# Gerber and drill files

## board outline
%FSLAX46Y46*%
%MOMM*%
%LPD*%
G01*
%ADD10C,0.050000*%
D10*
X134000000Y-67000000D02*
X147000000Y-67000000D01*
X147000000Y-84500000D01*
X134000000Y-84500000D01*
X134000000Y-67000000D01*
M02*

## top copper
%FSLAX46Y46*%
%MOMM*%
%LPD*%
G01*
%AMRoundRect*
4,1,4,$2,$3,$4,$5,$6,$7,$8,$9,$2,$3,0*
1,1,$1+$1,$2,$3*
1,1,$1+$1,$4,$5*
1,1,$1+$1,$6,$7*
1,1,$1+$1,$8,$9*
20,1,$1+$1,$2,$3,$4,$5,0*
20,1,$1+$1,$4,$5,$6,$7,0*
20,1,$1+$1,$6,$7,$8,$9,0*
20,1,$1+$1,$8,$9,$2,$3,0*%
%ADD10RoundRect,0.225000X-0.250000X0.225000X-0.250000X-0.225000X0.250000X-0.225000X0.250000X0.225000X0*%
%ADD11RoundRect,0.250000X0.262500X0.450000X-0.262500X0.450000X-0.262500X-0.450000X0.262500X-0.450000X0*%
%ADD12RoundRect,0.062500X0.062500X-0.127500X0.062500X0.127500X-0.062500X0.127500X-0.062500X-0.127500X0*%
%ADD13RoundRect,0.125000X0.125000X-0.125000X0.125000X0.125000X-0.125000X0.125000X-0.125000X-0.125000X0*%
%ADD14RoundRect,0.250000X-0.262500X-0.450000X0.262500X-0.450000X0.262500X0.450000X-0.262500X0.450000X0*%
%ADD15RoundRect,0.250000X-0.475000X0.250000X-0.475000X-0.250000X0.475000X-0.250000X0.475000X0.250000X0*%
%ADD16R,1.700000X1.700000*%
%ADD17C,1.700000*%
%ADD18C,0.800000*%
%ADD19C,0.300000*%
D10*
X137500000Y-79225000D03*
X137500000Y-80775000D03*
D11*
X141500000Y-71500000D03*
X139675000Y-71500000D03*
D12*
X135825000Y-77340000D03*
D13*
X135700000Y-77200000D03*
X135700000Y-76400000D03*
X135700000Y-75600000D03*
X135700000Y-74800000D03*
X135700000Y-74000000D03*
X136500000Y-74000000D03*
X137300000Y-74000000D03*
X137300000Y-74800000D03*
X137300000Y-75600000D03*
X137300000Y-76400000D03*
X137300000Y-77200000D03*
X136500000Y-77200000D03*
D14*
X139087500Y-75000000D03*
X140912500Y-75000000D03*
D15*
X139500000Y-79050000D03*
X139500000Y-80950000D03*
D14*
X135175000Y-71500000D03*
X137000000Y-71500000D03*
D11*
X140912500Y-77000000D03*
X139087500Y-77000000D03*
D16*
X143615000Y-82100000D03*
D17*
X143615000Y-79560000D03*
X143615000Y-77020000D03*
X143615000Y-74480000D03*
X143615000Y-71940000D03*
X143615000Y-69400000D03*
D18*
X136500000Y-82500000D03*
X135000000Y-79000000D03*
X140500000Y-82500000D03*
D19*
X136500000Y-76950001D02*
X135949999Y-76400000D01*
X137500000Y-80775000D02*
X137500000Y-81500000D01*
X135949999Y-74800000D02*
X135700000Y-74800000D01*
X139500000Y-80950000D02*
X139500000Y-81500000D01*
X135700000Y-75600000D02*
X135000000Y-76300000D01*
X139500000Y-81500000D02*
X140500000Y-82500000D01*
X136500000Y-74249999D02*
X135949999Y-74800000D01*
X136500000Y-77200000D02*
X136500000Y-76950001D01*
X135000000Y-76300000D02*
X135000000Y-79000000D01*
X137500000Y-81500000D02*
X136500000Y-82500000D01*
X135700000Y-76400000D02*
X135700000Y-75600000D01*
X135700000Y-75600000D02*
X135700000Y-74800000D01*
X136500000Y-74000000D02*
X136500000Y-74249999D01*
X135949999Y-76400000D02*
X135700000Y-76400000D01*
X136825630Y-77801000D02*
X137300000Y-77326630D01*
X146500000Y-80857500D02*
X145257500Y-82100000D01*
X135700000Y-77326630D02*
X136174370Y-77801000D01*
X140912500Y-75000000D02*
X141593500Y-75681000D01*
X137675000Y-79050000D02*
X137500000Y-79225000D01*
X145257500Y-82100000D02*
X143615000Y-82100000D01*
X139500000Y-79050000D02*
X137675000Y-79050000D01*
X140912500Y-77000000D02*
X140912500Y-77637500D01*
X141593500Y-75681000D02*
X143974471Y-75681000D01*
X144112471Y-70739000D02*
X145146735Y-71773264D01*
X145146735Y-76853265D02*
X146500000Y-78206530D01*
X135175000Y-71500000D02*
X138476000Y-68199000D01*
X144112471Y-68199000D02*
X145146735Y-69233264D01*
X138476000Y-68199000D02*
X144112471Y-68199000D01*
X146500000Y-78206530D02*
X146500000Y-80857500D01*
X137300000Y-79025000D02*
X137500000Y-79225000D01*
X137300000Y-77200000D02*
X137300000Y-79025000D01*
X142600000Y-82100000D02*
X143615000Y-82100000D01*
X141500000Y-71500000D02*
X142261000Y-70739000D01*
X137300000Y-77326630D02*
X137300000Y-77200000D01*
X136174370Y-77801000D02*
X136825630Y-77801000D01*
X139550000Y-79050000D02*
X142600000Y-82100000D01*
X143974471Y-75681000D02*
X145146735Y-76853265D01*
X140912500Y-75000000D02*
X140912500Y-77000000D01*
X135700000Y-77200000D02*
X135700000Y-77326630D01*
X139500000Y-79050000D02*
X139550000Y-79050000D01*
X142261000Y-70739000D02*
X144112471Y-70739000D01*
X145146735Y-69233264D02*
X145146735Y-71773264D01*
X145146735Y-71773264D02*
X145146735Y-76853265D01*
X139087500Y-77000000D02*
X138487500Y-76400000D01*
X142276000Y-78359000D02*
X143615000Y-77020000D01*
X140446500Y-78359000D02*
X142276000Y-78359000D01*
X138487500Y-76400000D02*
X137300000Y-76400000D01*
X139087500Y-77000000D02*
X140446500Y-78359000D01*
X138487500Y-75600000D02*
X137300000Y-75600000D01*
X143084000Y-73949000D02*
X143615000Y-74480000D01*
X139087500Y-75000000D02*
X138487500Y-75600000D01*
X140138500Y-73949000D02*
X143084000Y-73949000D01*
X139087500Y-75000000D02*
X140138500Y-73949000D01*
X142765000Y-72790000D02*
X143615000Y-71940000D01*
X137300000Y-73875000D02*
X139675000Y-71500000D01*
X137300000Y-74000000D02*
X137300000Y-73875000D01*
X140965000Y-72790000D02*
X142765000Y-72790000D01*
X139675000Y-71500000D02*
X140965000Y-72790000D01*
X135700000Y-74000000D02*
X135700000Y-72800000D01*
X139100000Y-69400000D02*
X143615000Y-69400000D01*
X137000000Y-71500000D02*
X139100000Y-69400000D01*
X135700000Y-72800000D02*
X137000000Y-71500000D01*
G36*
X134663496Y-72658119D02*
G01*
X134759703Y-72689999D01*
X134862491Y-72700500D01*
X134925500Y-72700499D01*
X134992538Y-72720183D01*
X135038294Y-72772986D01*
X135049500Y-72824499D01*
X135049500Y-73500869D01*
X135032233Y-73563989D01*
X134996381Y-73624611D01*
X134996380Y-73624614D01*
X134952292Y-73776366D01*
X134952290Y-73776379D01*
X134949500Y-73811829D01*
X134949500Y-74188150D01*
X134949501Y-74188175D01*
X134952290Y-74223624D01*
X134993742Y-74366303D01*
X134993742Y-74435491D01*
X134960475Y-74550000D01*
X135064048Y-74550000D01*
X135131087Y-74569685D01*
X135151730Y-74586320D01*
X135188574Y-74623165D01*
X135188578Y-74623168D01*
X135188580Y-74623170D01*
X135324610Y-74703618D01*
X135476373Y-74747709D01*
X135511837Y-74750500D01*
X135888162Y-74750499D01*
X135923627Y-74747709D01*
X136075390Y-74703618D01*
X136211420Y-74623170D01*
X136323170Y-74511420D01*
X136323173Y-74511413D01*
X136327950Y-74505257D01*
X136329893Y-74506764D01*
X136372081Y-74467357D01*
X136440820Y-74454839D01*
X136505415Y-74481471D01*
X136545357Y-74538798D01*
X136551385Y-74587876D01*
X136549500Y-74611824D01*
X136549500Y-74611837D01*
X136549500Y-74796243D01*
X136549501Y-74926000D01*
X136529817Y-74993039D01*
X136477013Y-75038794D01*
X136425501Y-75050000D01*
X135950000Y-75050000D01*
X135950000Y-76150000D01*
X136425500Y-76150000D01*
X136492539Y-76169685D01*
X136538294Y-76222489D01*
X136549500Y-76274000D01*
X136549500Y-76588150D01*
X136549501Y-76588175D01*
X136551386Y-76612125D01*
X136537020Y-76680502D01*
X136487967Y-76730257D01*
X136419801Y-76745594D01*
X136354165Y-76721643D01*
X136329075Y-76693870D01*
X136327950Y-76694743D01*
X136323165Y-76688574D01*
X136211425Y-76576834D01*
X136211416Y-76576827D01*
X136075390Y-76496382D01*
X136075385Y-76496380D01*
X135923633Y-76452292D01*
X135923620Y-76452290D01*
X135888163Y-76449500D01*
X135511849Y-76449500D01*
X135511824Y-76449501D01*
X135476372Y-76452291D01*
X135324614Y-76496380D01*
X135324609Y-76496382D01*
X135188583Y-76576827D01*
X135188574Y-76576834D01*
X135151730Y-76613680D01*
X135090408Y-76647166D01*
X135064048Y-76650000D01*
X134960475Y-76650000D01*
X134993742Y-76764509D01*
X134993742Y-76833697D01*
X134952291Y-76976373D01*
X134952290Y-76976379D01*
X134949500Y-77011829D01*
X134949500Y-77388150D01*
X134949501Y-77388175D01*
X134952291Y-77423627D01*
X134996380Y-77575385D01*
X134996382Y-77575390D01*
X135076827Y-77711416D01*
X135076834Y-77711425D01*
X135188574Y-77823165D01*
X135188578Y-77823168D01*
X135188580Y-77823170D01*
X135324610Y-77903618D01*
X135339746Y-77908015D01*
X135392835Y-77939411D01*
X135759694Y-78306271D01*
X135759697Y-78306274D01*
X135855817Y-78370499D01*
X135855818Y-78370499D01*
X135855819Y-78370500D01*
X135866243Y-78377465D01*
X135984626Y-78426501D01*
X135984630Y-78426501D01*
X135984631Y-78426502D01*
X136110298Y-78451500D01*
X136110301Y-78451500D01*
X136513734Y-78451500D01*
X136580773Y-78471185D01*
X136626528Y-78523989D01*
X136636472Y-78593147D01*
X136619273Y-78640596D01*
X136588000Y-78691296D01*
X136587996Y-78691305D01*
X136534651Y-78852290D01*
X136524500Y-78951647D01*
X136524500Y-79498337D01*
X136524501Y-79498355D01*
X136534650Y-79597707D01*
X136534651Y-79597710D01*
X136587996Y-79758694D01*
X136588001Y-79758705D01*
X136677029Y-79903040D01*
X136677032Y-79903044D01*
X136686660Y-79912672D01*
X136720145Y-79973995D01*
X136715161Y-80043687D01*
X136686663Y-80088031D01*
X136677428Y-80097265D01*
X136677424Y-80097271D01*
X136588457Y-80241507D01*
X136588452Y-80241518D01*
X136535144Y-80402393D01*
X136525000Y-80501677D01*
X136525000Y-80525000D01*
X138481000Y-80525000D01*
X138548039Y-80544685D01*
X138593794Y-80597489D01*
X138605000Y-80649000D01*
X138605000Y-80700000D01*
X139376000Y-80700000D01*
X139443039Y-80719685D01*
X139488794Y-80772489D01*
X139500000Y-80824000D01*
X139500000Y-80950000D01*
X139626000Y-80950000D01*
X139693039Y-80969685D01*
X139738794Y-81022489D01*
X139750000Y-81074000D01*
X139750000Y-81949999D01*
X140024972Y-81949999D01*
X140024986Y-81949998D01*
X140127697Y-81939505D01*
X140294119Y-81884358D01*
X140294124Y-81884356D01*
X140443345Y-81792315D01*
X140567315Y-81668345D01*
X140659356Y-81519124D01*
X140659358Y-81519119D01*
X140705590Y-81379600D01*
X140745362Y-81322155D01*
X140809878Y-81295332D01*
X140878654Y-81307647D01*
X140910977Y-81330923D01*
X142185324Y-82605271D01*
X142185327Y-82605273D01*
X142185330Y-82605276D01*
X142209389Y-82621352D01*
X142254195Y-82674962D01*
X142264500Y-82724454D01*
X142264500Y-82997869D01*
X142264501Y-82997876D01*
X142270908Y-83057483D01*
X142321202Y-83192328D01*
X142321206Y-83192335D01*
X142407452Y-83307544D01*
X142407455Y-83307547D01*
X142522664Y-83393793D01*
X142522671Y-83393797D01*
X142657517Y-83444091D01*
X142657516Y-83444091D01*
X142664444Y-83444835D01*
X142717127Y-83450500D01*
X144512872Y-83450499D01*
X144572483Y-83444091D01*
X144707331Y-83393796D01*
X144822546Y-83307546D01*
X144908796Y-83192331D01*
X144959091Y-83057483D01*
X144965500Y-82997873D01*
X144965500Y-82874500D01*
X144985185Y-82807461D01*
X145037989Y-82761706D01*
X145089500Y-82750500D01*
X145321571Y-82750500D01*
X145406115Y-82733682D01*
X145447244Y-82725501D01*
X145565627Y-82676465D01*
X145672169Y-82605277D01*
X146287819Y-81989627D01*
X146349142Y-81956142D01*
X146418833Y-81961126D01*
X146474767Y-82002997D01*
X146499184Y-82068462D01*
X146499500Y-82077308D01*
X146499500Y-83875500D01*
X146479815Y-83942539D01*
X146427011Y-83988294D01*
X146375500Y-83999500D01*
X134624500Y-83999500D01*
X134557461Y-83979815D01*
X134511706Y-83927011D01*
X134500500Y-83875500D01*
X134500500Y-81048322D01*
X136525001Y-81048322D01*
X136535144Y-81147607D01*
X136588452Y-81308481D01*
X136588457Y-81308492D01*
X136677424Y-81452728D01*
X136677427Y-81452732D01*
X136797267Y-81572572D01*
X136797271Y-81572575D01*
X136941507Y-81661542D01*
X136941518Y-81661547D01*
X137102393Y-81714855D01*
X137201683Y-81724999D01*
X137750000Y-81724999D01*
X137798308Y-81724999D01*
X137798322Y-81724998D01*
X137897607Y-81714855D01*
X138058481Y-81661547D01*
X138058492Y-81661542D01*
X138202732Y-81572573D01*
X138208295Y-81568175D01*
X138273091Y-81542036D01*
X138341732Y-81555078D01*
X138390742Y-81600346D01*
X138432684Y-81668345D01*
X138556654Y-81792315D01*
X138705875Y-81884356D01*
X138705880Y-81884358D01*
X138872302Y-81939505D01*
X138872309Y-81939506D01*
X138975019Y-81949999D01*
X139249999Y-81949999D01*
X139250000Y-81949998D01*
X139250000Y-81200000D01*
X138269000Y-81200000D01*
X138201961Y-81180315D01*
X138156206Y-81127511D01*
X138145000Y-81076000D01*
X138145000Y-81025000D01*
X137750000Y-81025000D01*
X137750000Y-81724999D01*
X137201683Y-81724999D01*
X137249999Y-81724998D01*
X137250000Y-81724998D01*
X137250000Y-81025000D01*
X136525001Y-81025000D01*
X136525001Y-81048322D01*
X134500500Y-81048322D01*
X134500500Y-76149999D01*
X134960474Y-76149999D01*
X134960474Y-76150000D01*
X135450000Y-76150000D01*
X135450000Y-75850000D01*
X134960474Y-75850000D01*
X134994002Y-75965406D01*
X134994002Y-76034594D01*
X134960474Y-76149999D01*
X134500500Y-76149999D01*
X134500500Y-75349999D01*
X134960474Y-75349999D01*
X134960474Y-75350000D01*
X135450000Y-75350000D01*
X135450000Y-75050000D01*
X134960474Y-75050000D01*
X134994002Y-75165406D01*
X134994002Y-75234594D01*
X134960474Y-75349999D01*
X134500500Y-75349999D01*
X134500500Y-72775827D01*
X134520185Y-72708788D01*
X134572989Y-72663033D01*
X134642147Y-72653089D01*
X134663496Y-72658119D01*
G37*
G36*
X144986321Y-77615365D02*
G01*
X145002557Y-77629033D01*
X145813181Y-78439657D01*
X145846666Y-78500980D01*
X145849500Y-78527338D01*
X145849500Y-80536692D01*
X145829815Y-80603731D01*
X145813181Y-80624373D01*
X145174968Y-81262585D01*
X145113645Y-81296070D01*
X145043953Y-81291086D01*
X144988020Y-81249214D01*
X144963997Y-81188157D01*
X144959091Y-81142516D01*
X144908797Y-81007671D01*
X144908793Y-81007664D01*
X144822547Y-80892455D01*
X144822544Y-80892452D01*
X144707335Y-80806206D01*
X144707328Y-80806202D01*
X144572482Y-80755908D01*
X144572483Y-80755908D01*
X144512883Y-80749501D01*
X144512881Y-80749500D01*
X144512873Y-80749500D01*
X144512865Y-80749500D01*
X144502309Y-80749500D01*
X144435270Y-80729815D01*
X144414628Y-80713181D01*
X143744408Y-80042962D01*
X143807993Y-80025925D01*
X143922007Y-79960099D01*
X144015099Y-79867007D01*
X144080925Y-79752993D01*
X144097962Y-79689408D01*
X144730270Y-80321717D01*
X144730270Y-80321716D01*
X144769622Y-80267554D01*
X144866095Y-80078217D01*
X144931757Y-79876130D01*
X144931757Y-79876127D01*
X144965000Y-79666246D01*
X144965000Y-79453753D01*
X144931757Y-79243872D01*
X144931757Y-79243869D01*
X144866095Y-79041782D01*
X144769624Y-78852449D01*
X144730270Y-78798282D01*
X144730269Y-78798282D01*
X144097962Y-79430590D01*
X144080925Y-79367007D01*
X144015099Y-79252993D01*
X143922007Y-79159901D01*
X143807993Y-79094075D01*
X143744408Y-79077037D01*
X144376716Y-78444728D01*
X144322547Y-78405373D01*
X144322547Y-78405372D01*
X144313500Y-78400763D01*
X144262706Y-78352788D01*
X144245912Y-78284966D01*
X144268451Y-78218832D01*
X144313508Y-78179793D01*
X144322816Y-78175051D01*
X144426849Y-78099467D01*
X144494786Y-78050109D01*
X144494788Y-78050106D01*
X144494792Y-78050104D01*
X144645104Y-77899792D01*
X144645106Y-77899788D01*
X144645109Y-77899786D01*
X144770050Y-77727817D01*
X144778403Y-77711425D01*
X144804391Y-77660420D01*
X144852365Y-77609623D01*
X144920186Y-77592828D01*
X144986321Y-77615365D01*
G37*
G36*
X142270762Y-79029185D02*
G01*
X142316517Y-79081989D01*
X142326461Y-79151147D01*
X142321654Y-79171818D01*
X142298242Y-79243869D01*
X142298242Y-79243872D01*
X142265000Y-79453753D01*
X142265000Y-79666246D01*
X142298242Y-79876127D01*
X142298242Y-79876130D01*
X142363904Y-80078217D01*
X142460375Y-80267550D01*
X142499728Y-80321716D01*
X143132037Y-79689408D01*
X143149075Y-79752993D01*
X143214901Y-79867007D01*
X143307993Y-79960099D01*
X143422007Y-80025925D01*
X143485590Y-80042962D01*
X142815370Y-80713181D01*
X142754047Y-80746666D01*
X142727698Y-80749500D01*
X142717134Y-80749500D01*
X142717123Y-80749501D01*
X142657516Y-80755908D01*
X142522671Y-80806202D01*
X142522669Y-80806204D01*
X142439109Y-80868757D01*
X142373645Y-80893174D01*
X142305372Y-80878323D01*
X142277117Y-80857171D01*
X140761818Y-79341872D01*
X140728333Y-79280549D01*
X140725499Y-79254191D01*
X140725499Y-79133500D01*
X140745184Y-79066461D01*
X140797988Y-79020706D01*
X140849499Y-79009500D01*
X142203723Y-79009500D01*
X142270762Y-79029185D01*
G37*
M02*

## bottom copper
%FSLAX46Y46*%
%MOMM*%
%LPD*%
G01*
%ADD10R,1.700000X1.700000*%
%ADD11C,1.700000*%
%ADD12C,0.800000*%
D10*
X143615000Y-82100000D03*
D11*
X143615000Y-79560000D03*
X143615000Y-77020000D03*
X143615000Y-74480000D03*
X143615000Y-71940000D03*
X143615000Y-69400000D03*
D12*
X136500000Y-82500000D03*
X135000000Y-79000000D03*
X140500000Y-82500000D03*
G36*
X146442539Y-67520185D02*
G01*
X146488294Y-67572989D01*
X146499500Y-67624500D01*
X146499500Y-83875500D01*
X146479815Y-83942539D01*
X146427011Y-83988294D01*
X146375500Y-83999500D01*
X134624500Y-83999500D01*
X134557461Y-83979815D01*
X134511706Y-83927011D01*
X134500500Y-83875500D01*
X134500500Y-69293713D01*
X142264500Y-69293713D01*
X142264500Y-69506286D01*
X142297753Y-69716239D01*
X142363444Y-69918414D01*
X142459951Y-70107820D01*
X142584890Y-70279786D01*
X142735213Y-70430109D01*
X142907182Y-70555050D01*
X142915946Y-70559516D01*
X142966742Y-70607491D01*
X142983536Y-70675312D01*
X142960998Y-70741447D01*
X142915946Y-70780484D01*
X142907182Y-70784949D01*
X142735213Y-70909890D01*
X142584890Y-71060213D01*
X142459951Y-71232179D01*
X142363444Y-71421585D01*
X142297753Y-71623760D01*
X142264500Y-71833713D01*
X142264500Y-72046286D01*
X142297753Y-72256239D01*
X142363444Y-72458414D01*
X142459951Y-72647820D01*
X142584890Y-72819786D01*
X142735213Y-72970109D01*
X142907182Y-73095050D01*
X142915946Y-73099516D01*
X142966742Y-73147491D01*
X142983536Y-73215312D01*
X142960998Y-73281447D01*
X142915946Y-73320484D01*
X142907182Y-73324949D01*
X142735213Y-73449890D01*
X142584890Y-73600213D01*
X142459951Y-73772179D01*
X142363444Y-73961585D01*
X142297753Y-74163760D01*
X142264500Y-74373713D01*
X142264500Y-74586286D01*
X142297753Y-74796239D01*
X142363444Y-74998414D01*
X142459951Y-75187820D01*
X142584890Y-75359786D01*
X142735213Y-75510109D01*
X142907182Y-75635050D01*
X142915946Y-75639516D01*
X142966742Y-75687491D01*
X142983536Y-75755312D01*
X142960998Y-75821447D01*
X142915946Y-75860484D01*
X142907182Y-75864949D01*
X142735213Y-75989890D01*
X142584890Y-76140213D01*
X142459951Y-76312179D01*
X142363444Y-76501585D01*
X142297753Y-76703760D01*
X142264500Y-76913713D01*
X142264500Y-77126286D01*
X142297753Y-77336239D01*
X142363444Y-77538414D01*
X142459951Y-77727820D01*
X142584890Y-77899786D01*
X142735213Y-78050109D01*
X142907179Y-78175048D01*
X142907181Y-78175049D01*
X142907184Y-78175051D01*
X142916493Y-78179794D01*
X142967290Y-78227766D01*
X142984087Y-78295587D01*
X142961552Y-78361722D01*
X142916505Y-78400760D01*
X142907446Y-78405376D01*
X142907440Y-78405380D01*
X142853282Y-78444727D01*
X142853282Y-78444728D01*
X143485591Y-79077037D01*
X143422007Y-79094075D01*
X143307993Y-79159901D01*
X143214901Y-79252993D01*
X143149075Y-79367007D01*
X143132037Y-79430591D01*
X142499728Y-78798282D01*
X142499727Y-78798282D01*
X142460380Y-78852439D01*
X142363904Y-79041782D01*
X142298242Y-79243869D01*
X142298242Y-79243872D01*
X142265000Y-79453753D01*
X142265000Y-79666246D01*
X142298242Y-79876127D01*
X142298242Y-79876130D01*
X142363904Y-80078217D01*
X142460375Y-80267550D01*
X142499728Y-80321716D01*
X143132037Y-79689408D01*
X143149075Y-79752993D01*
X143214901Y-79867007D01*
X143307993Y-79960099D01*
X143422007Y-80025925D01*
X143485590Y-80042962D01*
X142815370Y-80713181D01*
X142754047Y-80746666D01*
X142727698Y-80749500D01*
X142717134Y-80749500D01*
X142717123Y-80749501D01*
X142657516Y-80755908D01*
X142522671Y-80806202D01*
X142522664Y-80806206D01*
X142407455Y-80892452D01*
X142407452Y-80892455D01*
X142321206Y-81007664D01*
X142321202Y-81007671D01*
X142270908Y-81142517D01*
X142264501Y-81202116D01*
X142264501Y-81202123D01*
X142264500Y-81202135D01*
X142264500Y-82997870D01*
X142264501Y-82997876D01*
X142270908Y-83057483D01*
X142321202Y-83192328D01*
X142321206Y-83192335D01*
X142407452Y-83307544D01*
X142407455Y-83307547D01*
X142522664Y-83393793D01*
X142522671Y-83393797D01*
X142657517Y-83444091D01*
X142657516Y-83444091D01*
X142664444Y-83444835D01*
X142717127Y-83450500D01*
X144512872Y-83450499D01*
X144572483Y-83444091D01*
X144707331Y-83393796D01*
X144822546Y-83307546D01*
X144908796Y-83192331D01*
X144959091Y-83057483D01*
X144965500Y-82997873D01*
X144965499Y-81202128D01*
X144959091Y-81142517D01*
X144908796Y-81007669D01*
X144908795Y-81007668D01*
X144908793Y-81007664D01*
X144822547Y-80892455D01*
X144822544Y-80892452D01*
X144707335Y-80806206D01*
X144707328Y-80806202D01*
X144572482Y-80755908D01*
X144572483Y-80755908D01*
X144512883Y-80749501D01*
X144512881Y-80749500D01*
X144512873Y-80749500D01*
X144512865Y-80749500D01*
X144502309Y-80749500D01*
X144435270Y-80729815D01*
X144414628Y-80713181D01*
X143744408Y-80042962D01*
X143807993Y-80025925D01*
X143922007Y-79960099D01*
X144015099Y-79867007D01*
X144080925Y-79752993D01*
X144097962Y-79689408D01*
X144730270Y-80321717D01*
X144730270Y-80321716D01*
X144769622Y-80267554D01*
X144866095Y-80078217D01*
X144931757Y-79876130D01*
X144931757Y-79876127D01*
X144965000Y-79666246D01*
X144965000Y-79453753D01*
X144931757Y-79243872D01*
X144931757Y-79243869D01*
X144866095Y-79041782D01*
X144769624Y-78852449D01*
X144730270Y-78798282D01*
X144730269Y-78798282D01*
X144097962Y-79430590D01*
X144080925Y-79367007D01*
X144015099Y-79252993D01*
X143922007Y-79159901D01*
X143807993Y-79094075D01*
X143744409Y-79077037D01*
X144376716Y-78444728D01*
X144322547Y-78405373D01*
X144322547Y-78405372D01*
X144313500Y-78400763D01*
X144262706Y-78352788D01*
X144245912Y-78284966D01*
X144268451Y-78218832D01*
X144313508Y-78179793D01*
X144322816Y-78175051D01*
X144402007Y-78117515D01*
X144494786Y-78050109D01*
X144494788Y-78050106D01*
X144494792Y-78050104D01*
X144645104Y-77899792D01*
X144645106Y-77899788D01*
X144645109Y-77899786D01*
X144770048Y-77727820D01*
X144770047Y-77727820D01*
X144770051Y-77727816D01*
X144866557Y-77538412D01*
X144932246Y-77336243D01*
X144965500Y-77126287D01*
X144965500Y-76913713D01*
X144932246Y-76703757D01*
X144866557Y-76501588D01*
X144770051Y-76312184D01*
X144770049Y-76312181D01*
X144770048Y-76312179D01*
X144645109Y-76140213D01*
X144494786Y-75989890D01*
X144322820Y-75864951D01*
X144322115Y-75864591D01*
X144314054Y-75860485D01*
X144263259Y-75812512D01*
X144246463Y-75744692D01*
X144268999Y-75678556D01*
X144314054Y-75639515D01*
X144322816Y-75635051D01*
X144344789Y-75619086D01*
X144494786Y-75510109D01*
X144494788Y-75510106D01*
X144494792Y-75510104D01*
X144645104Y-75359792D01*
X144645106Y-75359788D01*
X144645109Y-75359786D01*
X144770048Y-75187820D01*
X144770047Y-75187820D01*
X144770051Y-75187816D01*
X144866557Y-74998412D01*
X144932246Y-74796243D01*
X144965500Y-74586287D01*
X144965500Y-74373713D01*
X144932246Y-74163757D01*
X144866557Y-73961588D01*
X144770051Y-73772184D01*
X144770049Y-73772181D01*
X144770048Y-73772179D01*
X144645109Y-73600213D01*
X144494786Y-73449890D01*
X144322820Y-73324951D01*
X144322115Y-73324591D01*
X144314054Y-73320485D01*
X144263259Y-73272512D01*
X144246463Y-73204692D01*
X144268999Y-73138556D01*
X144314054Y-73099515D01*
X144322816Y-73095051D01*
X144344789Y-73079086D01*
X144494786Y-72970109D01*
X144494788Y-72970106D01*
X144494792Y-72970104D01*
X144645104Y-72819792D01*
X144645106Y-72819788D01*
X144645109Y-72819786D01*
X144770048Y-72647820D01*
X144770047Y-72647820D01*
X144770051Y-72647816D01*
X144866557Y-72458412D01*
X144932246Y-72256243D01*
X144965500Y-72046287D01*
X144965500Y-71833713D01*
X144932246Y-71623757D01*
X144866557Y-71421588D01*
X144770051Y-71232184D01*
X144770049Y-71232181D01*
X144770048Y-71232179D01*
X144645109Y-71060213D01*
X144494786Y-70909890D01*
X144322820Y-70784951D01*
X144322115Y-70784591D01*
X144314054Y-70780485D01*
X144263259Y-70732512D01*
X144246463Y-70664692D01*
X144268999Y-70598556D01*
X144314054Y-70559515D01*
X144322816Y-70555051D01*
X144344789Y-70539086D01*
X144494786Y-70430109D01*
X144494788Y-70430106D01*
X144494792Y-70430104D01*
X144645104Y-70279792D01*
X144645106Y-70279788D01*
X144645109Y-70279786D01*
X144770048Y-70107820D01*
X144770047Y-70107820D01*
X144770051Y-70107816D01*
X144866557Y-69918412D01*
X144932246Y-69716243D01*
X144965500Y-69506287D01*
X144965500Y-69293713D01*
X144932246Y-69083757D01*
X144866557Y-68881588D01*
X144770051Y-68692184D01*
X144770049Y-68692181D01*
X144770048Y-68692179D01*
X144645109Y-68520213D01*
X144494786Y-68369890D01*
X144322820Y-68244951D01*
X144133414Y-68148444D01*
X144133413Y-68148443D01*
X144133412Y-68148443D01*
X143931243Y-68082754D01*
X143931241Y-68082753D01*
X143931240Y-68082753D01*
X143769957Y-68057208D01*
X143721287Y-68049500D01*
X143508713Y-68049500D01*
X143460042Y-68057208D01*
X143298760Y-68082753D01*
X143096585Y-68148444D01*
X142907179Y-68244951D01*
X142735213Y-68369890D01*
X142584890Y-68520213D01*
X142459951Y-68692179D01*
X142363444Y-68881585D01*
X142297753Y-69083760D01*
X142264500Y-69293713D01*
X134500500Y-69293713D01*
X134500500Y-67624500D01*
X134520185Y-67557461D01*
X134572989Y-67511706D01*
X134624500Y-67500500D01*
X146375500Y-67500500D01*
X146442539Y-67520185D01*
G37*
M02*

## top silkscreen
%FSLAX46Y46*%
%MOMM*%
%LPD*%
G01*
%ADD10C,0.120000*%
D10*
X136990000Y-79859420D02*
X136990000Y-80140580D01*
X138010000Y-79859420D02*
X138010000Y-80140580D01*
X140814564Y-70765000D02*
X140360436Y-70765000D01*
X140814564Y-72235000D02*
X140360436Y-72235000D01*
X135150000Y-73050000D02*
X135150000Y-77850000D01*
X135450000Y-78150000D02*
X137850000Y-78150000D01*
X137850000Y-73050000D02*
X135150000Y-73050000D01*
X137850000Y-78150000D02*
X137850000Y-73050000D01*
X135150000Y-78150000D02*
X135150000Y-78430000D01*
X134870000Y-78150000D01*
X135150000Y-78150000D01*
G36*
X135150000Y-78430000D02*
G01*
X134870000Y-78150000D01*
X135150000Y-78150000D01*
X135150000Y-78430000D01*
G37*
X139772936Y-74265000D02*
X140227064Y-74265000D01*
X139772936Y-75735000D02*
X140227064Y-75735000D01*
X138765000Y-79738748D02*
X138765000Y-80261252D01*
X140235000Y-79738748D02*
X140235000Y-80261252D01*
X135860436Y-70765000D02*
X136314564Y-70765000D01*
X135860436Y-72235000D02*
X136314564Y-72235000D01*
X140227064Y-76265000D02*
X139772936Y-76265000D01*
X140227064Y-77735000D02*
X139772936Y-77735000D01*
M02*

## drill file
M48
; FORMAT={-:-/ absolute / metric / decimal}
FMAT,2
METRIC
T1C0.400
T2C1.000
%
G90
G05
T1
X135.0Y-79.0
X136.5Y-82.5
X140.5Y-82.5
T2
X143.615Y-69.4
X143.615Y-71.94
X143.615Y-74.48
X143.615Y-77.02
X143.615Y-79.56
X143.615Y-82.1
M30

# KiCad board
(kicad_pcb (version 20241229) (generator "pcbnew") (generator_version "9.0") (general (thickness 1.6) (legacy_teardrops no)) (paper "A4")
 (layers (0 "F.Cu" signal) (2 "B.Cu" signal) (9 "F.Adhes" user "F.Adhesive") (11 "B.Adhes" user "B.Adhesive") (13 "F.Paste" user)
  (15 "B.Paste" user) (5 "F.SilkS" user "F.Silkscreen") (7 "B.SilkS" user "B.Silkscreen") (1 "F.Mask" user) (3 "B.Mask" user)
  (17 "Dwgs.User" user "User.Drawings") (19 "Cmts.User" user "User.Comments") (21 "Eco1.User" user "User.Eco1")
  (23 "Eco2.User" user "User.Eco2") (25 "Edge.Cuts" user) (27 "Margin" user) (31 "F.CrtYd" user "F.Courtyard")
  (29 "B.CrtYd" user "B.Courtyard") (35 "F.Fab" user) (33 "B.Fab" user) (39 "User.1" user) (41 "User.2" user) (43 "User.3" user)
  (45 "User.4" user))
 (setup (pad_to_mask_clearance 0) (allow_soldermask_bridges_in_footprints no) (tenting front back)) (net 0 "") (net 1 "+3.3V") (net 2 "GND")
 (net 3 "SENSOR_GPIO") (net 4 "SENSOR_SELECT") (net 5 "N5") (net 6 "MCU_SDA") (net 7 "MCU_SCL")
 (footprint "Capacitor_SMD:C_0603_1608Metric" (layer "F.Cu") (at 137.5 80 -90)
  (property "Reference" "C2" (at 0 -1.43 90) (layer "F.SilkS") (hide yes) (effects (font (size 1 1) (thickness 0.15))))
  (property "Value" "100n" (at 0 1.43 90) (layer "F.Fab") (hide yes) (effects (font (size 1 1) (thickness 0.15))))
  (fp_line (start -0.14058 0.51) (end 0.14058 0.51) (stroke (width 0.12) (type solid)) (layer "F.SilkS"))
  (fp_line (start -0.14058 -0.51) (end 0.14058 -0.51) (stroke (width 0.12) (type solid)) (layer "F.SilkS"))
  (pad "1" smd roundrect (at -0.775 0 270) (size 0.9 0.95) (layers "F.Cu" "F.Mask" "F.Paste") (roundrect_rratio 0.25) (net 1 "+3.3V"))
  (pad "2" smd roundrect (at 0.775 0 270) (size 0.9 0.95) (layers "F.Cu" "F.Mask" "F.Paste") (roundrect_rratio 0.25) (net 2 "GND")))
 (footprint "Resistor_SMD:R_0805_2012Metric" (layer "F.Cu") (at 140.5875 71.5 180)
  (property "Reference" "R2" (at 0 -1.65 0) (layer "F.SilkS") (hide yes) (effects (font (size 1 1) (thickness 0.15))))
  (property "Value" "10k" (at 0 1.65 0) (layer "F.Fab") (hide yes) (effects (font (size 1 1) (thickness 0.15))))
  (fp_line (start -0.227064 0.735) (end 0.227064 0.735) (stroke (width 0.12) (type solid)) (layer "F.SilkS"))
  (fp_line (start -0.227064 -0.735) (end 0.227064 -0.735) (stroke (width 0.12) (type solid)) (layer "F.SilkS"))
  (pad "1" smd roundrect (at -0.9125 0 180) (size 1.025 1.4) (layers "F.Cu" "F.Mask" "F.Paste") (roundrect_rratio 0.243902) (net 1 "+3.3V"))
  (pad "2" smd roundrect (at 0.9125 0 180) (size 1.025 1.4) (layers "F.Cu" "F.Mask" "F.Paste") (roundrect_rratio 0.243902)
   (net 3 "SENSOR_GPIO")))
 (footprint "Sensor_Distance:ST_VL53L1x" (layer "F.Cu") (at 136.5 75.6 90)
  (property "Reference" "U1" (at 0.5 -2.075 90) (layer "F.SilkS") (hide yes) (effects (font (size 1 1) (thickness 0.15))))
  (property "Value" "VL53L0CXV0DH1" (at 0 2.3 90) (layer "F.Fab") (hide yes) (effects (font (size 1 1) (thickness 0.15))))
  (fp_line (start 2.55 -1.35) (end -2.25 -1.35) (stroke (width 0.12) (type solid)) (layer "F.SilkS"))
  (fp_line (start -2.55 -1.05) (end -2.55 1.35) (stroke (width 0.12) (type solid)) (layer "F.SilkS"))
  (fp_line (start 2.55 1.35) (end 2.55 -1.35) (stroke (width 0.12) (type solid)) (layer "F.SilkS"))
  (fp_line (start -2.55 1.35) (end 2.55 1.35) (stroke (width 0.12) (type solid)) (layer "F.SilkS"))
  (fp_poly
   (pts (xy -2.55 -1.35) (xy -2.83 -1.35) (xy -2.55 -1.63) (xy -2.55 -1.35)) (stroke (width 0.12) (type solid)) (fill yes) (layer "F.SilkS"))
  (pad "1" smd roundrect (at -1.74 -0.675 90) (size 0.38 0.25) (layers "F.Cu" "F.Mask" "F.Paste") (roundrect_rratio 0.25) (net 1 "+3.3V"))
  (pad "1" smd roundrect (at -1.6 -0.8 90) (size 0.5 0.5) (layers "F.Cu" "F.Mask" "F.Paste") (roundrect_rratio 0.25) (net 1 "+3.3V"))
  (pad "2" smd roundrect (at -0.8 -0.8 90) (size 0.5 0.5) (layers "F.Cu" "F.Mask" "F.Paste") (roundrect_rratio 0.25) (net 2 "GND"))
  (pad "3" smd roundrect (at 0 -0.8 90) (size 0.5 0.5) (layers "F.Cu" "F.Mask" "F.Paste") (roundrect_rratio 0.25) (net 2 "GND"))
  (pad "4" smd roundrect (at 0.8 -0.8 90) (size 0.5 0.5) (layers "F.Cu" "F.Mask" "F.Paste") (roundrect_rratio 0.25) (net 2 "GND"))
  (pad "5" smd roundrect (at 1.6 -0.8 90) (size 0.5 0.5) (layers "F.Cu" "F.Mask" "F.Paste") (roundrect_rratio 0.25) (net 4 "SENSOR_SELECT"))
  (pad "6" smd roundrect (at 1.6 0 90) (size 0.5 0.5) (layers "F.Cu" "F.Mask" "F.Paste") (roundrect_rratio 0.25) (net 2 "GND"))
  (pad "7" smd roundrect (at 1.6 0.8 90) (size 0.5 0.5) (layers "F.Cu" "F.Mask" "F.Paste") (roundrect_rratio 0.25) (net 3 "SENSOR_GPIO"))
  (pad "8" smd roundrect (at 0.8 0.8 90) (size 0.5 0.5) (layers "F.Cu" "F.Mask" "F.Paste") (roundrect_rratio 0.25) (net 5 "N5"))
  (pad "9" smd roundrect (at 0 0.8 90) (size 0.5 0.5) (layers "F.Cu" "F.Mask" "F.Paste") (roundrect_rratio 0.25) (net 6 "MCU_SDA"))
  (pad "10" smd roundrect (at -0.8 0.8 90) (size 0.5 0.5) (layers "F.Cu" "F.Mask" "F.Paste") (roundrect_rratio 0.25) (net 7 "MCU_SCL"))
  (pad "11" smd roundrect (at -1.6 0.8 90) (size 0.5 0.5) (layers "F.Cu" "F.Mask" "F.Paste") (roundrect_rratio 0.25) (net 1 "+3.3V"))
  (pad "12" smd roundrect (at -1.6 0 90) (size 0.5 0.5) (layers "F.Cu" "F.Mask" "F.Paste") (roundrect_rratio 0.25) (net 2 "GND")))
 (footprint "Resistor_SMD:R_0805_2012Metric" (layer "F.Cu") (at 140 75)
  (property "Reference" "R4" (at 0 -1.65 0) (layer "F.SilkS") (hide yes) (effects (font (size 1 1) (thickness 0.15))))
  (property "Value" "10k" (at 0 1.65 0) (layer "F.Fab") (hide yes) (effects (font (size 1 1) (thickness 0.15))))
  (fp_line (start -0.227064 -0.735) (end 0.227064 -0.735) (stroke (width 0.12) (type solid)) (layer "F.SilkS"))
  (fp_line (start -0.227064 0.735) (end 0.227064 0.735) (stroke (width 0.12) (type solid)) (layer "F.SilkS"))
  (pad "1" smd roundrect (at -0.9125 0) (size 1.025 1.4) (layers "F.Cu" "F.Mask" "F.Paste") (roundrect_rratio 0.243902) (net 6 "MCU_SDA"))
  (pad "2" smd roundrect (at 0.9125 0) (size 1.025 1.4) (layers "F.Cu" "F.Mask" "F.Paste") (roundrect_rratio 0.243902) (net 1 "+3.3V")))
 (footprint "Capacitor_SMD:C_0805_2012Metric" (layer "F.Cu") (at 139.5 80 -90)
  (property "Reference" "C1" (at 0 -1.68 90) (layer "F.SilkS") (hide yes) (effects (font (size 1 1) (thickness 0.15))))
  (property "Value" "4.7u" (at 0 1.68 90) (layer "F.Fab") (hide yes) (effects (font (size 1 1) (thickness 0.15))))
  (fp_line (start -0.261252 0.735) (end 0.261252 0.735) (stroke (width 0.12) (type solid)) (layer "F.SilkS"))
  (fp_line (start -0.261252 -0.735) (end 0.261252 -0.735) (stroke (width 0.12) (type solid)) (layer "F.SilkS"))
  (pad "1" smd roundrect (at -0.95 0 270) (size 1 1.45) (layers "F.Cu" "F.Mask" "F.Paste") (roundrect_rratio 0.25) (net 1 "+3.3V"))
  (pad "2" smd roundrect (at 0.95 0 270) (size 1 1.45) (layers "F.Cu" "F.Mask" "F.Paste") (roundrect_rratio 0.25) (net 2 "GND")))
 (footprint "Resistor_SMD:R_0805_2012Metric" (layer "F.Cu") (at 136.0875 71.5)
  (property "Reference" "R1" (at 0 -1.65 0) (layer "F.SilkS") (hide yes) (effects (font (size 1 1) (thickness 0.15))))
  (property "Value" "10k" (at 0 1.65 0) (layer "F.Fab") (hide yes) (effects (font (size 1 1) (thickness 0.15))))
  (fp_line (start -0.227064 -0.735) (end 0.227064 -0.735) (stroke (width 0.12) (type solid)) (layer "F.SilkS"))
  (fp_line (start -0.227064 0.735) (end 0.227064 0.735) (stroke (width 0.12) (type solid)) (layer "F.SilkS"))
  (pad "1" smd roundrect (at -0.9125 0) (size 1.025 1.4) (layers "F.Cu" "F.Mask" "F.Paste") (roundrect_rratio 0.243902) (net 1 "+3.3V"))
  (pad "2" smd roundrect (at 0.9125 0) (size 1.025 1.4) (layers "F.Cu" "F.Mask" "F.Paste") (roundrect_rratio 0.243902)
   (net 4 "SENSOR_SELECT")))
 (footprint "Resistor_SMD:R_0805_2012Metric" (layer "F.Cu") (at 140 77 180)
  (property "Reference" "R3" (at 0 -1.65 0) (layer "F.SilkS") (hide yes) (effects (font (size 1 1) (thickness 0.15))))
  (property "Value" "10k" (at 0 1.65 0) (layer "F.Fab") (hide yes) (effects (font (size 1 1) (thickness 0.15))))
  (fp_line (start -0.227064 0.735) (end 0.227064 0.735) (stroke (width 0.12) (type solid)) (layer "F.SilkS"))
  (fp_line (start -0.227064 -0.735) (end 0.227064 -0.735) (stroke (width 0.12) (type solid)) (layer "F.SilkS"))
  (pad "1" smd roundrect (at -0.9125 0 180) (size 1.025 1.4) (layers "F.Cu" "F.Mask" "F.Paste") (roundrect_rratio 0.243902) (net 1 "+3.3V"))
  (pad "2" smd roundrect (at 0.9125 0 180) (size 1.025 1.4) (layers "F.Cu" "F.Mask" "F.Paste") (roundrect_rratio 0.243902) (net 7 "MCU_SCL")))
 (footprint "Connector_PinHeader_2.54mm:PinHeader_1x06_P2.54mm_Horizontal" (layer "B.Cu") (at 143.615 82.1)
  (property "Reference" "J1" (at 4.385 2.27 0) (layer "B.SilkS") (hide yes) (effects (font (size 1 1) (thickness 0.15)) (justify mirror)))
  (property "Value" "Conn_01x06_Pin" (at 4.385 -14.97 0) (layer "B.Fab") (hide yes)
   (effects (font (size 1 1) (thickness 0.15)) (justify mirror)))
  (pad "1" thru_hole rect (at 0 0) (size 1.7 1.7) (drill 1) (layers "*.Cu" "*.Mask") (remove_unused_layers no) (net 1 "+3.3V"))
  (pad "2" thru_hole circle (at 0 -2.54) (size 1.7 1.7) (drill 1) (layers "*.Cu" "*.Mask") (remove_unused_layers no) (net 2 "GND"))
  (pad "3" thru_hole circle (at 0 -5.08) (size 1.7 1.7) (drill 1) (layers "*.Cu" "*.Mask") (remove_unused_layers no) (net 7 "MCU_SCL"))
  (pad "4" thru_hole circle (at 0 -7.62) (size 1.7 1.7) (drill 1) (layers "*.Cu" "*.Mask") (remove_unused_layers no) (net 6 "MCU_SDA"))
  (pad "5" thru_hole circle (at 0 -10.16) (size 1.7 1.7) (drill 1) (layers "*.Cu" "*.Mask") (remove_unused_layers no) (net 3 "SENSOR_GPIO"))
  (pad "6" thru_hole circle (at 0 -12.7) (size 1.7 1.7) (drill 1) (layers "*.Cu" "*.Mask") (remove_unused_layers no) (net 4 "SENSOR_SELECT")))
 (gr_rect (start 134 67) (end 147 84.5) (stroke (width 0.05) (type default)) (fill no) (layer "Edge.Cuts"))
 (segment (start 136.5 76.950001) (end 135.949999 76.4) (width 0.3) (layer "F.Cu") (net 2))
 (segment (start 137.5 80.775) (end 137.5 81.5) (width 0.3) (layer "F.Cu") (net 2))
 (segment (start 135.949999 74.8) (end 135.7 74.8) (width 0.3) (layer "F.Cu") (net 2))
 (segment (start 139.5 80.95) (end 139.5 81.5) (width 0.3) (layer "F.Cu") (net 2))
 (segment (start 135.7 75.6) (end 135 76.3) (width 0.3) (layer "F.Cu") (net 2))
 (segment (start 139.5 81.5) (end 140.5 82.5) (width 0.3) (layer "F.Cu") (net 2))
 (segment (start 136.5 74.249999) (end 135.949999 74.8) (width 0.3) (layer "F.Cu") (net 2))
 (segment (start 136.5 77.2) (end 136.5 76.950001) (width 0.3) (layer "F.Cu") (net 2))
 (segment (start 135 76.3) (end 135 79) (width 0.3) (layer "F.Cu") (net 2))
 (segment (start 137.5 81.5) (end 136.5 82.5) (width 0.3) (layer "F.Cu") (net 2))
 (segment (start 135.7 76.4) (end 135.7 75.6) (width 0.3) (layer "F.Cu") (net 2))
 (segment (start 135.7 75.6) (end 135.7 74.8) (width 0.3) (layer "F.Cu") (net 2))
 (segment (start 136.5 74) (end 136.5 74.249999) (width 0.3) (layer "F.Cu") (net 2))
 (segment (start 135.949999 76.4) (end 135.7 76.4) (width 0.3) (layer "F.Cu") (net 2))
 (via (at 136.5 82.5) (size 0.8) (drill 0.4) (layers "F.Cu" "B.Cu") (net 2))
 (via (at 135 79) (size 0.8) (drill 0.4) (layers "F.Cu" "B.Cu") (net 2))
 (via (at 140.5 82.5) (size 0.8) (drill 0.4) (layers "F.Cu" "B.Cu") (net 2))
 (segment (start 136.82563 77.801) (end 137.3 77.32663) (width 0.3) (layer "F.Cu") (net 1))
 (segment (start 146.5 80.8575) (end 145.2575 82.1) (width 0.3) (layer "F.Cu") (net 1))
 (segment (start 135.7 77.32663) (end 136.17437 77.801) (width 0.3) (layer "F.Cu") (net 1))
 (segment (start 140.9125 75) (end 141.5935 75.681) (width 0.3) (layer "F.Cu") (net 1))
 (segment (start 137.675 79.05) (end 137.5 79.225) (width 0.3) (layer "F.Cu") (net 1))
 (segment (start 145.2575 82.1) (end 143.615 82.1) (width 0.3) (layer "F.Cu") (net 1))
 (segment (start 139.5 79.05) (end 137.675 79.05) (width 0.3) (layer "F.Cu") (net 1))
 (segment (start 140.9125 77) (end 140.9125 77.6375) (width 0.3) (layer "F.Cu") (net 1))
 (segment (start 141.5935 75.681) (end 143.974471 75.681) (width 0.3) (layer "F.Cu") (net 1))
 (segment (start 144.112471 70.739) (end 145.146735 71.773264) (width 0.3) (layer "F.Cu") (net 1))
 (segment (start 145.146735 76.853265) (end 146.5 78.20653) (width 0.3) (layer "F.Cu") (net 1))
 (segment (start 135.175 71.5) (end 138.476 68.199) (width 0.3) (layer "F.Cu") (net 1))
 (segment (start 144.112471 68.199) (end 145.146735 69.233264) (width 0.3) (layer "F.Cu") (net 1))
 (segment (start 138.476 68.199) (end 144.112471 68.199) (width 0.3) (layer "F.Cu") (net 1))
 (segment (start 146.5 78.20653) (end 146.5 80.8575) (width 0.3) (layer "F.Cu") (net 1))
 (segment (start 137.3 79.025) (end 137.5 79.225) (width 0.3) (layer "F.Cu") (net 1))
 (segment (start 137.3 77.2) (end 137.3 79.025) (width 0.3) (layer "F.Cu") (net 1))
 (segment (start 142.6 82.1) (end 143.615 82.1) (width 0.3) (layer "F.Cu") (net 1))
 (segment (start 141.5 71.5) (end 142.261 70.739) (width 0.3) (layer "F.Cu") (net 1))
 (segment (start 137.3 77.32663) (end 137.3 77.2) (width 0.3) (layer "F.Cu") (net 1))
 (segment (start 136.17437 77.801) (end 136.82563 77.801) (width 0.3) (layer "F.Cu") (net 1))
 (segment (start 139.55 79.05) (end 142.6 82.1) (width 0.3) (layer "F.Cu") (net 1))
 (segment (start 143.974471 75.681) (end 145.146735 76.853265) (width 0.3) (layer "F.Cu") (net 1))
 (segment (start 140.9125 75) (end 140.9125 77) (width 0.3) (layer "F.Cu") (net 1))
 (segment (start 135.7 77.2) (end 135.7 77.32663) (width 0.3) (layer "F.Cu") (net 1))
 (segment (start 139.5 79.05) (end 139.55 79.05) (width 0.3) (layer "F.Cu") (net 1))
 (segment (start 142.261 70.739) (end 144.112471 70.739) (width 0.3) (layer "F.Cu") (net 1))
 (segment (start 145.146735 69.233264) (end 145.146735 71.773264) (width 0.3) (layer "F.Cu") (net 1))
 (segment (start 145.146735 71.773264) (end 145.146735 76.853265) (width 0.3) (layer "F.Cu") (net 1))
 (segment (start 139.0875 77) (end 138.4875 76.4) (width 0.3) (layer "F.Cu") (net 7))
 (segment (start 142.276 78.359) (end 143.615 77.02) (width 0.3) (layer "F.Cu") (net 7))
 (segment (start 140.4465 78.359) (end 142.276 78.359) (width 0.3) (layer "F.Cu") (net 7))
 (segment (start 138.4875 76.4) (end 137.3 76.4) (width 0.3) (layer "F.Cu") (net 7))
 (segment (start 139.0875 77) (end 140.4465 78.359) (width 0.3) (layer "F.Cu") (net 7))
 (segment (start 138.4875 75.6) (end 137.3 75.6) (width 0.3) (layer "F.Cu") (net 6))
 (segment (start 143.084 73.949) (end 143.615 74.48) (width 0.3) (layer "F.Cu") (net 6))
 (segment (start 139.0875 75) (end 138.4875 75.6) (width 0.3) (layer "F.Cu") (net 6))
 (segment (start 140.1385 73.949) (end 143.084 73.949) (width 0.3) (layer "F.Cu") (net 6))
 (segment (start 139.0875 75) (end 140.1385 73.949) (width 0.3) (layer "F.Cu") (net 6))
 (segment (start 142.765 72.79) (end 143.615 71.94) (width 0.3) (layer "F.Cu") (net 3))
 (segment (start 137.3 73.875) (end 139.675 71.5) (width 0.3) (layer "F.Cu") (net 3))
 (segment (start 137.3 74) (end 137.3 73.875) (width 0.3) (layer "F.Cu") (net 3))
 (segment (start 140.965 72.79) (end 142.765 72.79) (width 0.3) (layer "F.Cu") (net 3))
 (segment (start 139.675 71.5) (end 140.965 72.79) (width 0.3) (layer "F.Cu") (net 3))
 (segment (start 135.7 74) (end 135.7 72.8) (width 0.3) (layer "F.Cu") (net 4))
 (segment (start 139.1 69.4) (end 143.615 69.4) (width 0.3) (layer "F.Cu") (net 4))
 (segment (start 137 71.5) (end 139.1 69.4) (width 0.3) (layer "F.Cu") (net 4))
 (segment (start 135.7 72.8) (end 137 71.5) (width 0.3) (layer "F.Cu") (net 4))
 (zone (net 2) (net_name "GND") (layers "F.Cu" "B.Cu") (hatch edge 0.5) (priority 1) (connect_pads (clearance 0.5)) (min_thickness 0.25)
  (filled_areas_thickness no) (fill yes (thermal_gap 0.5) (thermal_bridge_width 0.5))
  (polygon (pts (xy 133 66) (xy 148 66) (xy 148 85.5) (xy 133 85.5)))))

